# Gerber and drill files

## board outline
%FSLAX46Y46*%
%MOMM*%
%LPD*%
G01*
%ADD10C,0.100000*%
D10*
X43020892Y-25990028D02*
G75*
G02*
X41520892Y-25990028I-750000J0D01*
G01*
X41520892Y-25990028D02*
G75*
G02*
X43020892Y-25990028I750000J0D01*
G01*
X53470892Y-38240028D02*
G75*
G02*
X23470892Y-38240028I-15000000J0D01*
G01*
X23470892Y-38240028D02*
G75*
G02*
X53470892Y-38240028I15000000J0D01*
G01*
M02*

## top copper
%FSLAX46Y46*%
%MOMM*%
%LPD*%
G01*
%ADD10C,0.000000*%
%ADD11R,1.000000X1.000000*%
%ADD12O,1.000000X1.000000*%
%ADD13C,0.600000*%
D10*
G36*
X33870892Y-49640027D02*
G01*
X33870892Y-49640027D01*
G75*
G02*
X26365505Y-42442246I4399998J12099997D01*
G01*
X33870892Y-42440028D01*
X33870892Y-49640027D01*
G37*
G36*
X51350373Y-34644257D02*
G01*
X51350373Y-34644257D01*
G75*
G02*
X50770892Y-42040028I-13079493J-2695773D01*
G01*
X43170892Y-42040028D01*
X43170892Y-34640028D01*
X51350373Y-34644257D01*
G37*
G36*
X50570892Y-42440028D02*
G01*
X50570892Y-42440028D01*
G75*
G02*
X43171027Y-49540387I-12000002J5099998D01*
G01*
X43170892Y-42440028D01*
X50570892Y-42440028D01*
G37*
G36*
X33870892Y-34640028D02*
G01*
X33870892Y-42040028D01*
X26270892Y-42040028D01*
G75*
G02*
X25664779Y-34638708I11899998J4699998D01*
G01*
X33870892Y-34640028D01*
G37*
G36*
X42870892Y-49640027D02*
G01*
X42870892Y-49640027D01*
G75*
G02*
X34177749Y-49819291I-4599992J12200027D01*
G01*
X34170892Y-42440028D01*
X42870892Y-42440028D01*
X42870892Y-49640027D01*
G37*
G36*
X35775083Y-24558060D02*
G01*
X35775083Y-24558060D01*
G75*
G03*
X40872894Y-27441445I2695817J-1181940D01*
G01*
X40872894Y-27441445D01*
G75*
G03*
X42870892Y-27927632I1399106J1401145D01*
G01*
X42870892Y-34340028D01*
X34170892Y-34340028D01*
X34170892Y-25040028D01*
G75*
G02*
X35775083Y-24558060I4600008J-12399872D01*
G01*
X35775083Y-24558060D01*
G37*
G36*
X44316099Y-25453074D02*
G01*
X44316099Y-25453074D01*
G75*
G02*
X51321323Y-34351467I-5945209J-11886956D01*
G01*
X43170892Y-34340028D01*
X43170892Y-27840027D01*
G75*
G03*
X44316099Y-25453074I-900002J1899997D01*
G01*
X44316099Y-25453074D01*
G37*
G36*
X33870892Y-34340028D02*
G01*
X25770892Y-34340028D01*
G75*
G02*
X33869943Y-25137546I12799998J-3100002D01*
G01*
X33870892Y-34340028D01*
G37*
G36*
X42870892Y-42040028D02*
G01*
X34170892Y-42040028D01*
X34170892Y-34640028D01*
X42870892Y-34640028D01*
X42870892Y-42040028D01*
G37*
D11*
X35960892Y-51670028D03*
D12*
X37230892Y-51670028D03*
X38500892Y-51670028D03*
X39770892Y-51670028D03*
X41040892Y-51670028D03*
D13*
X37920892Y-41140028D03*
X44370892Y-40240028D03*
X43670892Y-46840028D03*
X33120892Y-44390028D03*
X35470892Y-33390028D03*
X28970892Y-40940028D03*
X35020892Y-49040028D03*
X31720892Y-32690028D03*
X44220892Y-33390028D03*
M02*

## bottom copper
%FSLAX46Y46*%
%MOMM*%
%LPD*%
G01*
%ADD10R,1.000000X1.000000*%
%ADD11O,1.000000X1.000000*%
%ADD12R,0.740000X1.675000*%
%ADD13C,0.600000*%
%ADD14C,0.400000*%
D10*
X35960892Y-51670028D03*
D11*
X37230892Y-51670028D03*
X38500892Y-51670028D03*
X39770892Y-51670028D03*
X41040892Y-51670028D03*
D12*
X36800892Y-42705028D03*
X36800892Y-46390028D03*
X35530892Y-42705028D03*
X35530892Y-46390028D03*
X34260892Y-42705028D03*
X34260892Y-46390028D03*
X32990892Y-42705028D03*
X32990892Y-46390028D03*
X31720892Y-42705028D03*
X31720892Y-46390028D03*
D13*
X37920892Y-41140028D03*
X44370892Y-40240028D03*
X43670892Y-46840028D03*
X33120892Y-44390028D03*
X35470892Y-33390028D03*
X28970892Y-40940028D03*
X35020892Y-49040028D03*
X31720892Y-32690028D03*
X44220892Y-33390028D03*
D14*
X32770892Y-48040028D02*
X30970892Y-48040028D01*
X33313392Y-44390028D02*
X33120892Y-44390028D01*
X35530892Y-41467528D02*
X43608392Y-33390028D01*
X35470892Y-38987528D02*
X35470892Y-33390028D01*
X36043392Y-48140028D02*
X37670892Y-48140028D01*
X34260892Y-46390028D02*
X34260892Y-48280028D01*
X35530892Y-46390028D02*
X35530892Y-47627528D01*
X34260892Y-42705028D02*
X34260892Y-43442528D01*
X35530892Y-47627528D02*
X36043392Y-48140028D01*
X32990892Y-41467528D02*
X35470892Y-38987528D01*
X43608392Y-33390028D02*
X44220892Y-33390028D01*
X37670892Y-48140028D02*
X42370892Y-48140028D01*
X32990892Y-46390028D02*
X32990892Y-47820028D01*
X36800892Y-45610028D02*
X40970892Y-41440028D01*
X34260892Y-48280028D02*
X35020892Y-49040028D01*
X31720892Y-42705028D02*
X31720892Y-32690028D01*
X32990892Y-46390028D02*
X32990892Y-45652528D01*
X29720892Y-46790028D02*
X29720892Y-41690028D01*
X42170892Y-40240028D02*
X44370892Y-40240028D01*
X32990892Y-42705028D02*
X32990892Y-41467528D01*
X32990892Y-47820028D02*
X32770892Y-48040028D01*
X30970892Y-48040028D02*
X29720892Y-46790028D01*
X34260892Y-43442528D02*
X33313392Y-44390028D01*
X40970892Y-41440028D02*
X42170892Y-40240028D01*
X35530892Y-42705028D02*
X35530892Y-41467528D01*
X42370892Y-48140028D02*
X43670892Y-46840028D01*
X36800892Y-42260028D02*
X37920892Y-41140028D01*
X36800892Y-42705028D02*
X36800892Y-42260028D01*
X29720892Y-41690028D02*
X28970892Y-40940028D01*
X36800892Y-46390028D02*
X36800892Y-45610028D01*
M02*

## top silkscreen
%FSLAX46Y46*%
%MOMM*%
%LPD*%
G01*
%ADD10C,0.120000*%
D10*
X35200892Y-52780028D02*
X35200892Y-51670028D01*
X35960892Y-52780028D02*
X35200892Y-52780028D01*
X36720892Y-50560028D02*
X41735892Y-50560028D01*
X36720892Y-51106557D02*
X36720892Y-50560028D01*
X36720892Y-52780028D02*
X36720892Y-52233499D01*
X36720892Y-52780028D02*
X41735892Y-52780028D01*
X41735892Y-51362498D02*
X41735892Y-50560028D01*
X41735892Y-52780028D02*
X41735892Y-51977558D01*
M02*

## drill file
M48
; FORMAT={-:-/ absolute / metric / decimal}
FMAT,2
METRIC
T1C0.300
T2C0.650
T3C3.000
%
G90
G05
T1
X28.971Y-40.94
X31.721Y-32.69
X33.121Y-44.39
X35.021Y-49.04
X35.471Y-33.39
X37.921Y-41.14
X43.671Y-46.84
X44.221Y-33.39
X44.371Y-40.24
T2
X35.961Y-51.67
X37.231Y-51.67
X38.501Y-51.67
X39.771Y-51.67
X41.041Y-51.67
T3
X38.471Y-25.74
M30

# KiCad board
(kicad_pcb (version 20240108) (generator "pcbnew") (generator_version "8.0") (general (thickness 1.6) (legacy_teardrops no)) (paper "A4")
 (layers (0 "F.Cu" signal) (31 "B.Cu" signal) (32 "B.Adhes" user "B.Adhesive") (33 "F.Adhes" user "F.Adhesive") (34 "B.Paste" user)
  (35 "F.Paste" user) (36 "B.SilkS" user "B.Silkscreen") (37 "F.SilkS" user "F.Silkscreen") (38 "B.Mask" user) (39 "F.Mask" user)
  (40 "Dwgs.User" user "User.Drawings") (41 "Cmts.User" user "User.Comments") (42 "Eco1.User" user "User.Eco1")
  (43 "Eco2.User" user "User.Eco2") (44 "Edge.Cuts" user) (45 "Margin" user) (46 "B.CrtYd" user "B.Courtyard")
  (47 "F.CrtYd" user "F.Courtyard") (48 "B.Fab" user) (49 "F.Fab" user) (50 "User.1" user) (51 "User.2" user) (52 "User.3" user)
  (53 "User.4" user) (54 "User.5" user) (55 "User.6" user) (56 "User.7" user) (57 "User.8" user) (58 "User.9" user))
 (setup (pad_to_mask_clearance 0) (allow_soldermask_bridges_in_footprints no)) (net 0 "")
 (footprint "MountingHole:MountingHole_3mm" (layer "F.Cu") (at 38.470892 25.740028)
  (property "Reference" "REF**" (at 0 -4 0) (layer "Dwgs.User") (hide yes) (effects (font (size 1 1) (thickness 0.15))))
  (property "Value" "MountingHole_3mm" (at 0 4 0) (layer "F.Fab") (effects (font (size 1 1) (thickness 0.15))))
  (pad "" np_thru_hole circle (at 0 0) (size 3 3) (drill 3) (layers "*.Cu" "*.Mask")))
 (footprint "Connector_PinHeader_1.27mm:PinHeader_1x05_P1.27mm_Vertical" (layer "F.Cu") (at 35.960892 51.670028 90)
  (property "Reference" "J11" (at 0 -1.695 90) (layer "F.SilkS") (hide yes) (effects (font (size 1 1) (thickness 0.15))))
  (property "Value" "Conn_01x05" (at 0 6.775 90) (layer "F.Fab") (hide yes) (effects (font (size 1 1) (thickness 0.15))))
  (fp_line (start -1.11 -0.76) (end 0 -0.76) (stroke (width 0.12) (type solid)) (layer "F.SilkS"))
  (fp_line (start -1.11 0) (end -1.11 -0.76) (stroke (width 0.12) (type solid)) (layer "F.SilkS"))
  (fp_line (start 1.11 0.76) (end 1.11 5.775) (stroke (width 0.12) (type solid)) (layer "F.SilkS"))
  (fp_line (start 0.563471 0.76) (end 1.11 0.76) (stroke (width 0.12) (type solid)) (layer "F.SilkS"))
  (fp_line (start -1.11 0.76) (end -0.563471 0.76) (stroke (width 0.12) (type solid)) (layer "F.SilkS"))
  (fp_line (start -1.11 0.76) (end -1.11 5.775) (stroke (width 0.12) (type solid)) (layer "F.SilkS"))
  (fp_line (start 0.30753 5.775) (end 1.11 5.775) (stroke (width 0.12) (type solid)) (layer "F.SilkS"))
  (fp_line (start -1.11 5.775) (end -0.30753 5.775) (stroke (width 0.12) (type solid)) (layer "F.SilkS"))
  (pad "1" thru_hole rect (at 0 0 90) (size 1 1) (drill 0.65) (layers "*.Cu" "*.Mask") (remove_unused_layers no))
  (pad "2" thru_hole oval (at 0 1.27 90) (size 1 1) (drill 0.65) (layers "*.Cu" "*.Mask") (remove_unused_layers no))
  (pad "3" thru_hole oval (at 0 2.54 90) (size 1 1) (drill 0.65) (layers "*.Cu" "*.Mask") (remove_unused_layers no))
  (pad "4" thru_hole oval (at 0 3.81 90) (size 1 1) (drill 0.65) (layers "*.Cu" "*.Mask") (remove_unused_layers no))
  (pad "5" thru_hole oval (at 0 5.08 90) (size 1 1) (drill 0.65) (layers "*.Cu" "*.Mask") (remove_unused_layers no)))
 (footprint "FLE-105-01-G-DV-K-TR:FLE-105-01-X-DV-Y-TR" (layer "B.Cu") (at 34.260892 44.547528 180)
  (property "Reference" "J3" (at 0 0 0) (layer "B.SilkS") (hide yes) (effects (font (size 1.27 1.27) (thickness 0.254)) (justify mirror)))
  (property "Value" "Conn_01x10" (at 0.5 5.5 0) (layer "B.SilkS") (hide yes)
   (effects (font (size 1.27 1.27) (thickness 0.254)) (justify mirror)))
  (pad "1" smd rect (at -2.54 1.8425 180) (size 0.74 1.675) (layers "B.Cu" "B.Paste" "B.Mask"))
  (pad "2" smd rect (at -2.54 -1.8425 180) (size 0.74 1.675) (layers "B.Cu" "B.Paste" "B.Mask"))
  (pad "3" smd rect (at -1.27 1.8425 180) (size 0.74 1.675) (layers "B.Cu" "B.Paste" "B.Mask"))
  (pad "4" smd rect (at -1.27 -1.8425 180) (size 0.74 1.675) (layers "B.Cu" "B.Paste" "B.Mask"))
  (pad "5" smd rect (at 0 1.8425 180) (size 0.74 1.675) (layers "B.Cu" "B.Paste" "B.Mask"))
  (pad "6" smd rect (at 0 -1.8425 180) (size 0.74 1.675) (layers "B.Cu" "B.Paste" "B.Mask"))
  (pad "7" smd rect (at 1.27 1.8425 180) (size 0.74 1.675) (layers "B.Cu" "B.Paste" "B.Mask"))
  (pad "8" smd rect (at 1.27 -1.8425 180) (size 0.74 1.675) (layers "B.Cu" "B.Paste" "B.Mask"))
  (pad "9" smd rect (at 2.54 1.8425 180) (size 0.74 1.675) (layers "B.Cu" "B.Paste" "B.Mask"))
  (pad "10" smd rect (at 2.54 -1.8425 180) (size 0.74 1.675) (layers "B.Cu" "B.Paste" "B.Mask")))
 (gr_poly
  (pts (arc (start 26.365505 42.442246) (mid 29.359191 46.832582) (end 33.870892 49.640027)) (xy 33.870892 42.440028))
  (stroke (width 0) (type solid)) (fill solid) (layer "F.Cu"))
 (gr_poly
  (pts (xy 43.170892 42.040028) (xy 43.170892 34.640028)
   (arc (start 51.350373 34.644257) (mid 51.584487 38.383188) (end 50.770892 42.040028)))
  (stroke (width 0) (type solid)) (fill solid) (layer "F.Cu"))
 (gr_poly
  (pts (arc (start 50.570892 42.440028) (mid 47.598344 46.748275) (end 43.171027 49.540387)) (xy 43.170892 42.440028))
  (stroke (width 0) (type solid)) (fill solid) (layer "F.Cu"))
 (gr_poly
  (pts
   (arc (start 25.664779 34.638708) (mid 25.41905 38.384309) (end 26.270892 42.040028)) (xy 33.870892 42.040028) (xy 33.870892 34.640028))
  (stroke (width 0) (type solid)) (fill solid) (layer "F.Cu"))
 (gr_poly
  (pts
   (arc (start 34.177749 49.819291) (mid 38.539704 50.475661) (end 42.870892 49.640027)) (xy 42.870892 42.440028) (xy 34.170892 42.440028))
  (stroke (width 0) (type solid)) (fill solid) (layer "F.Cu"))
 (gr_poly
  (pts
   (arc (start 35.775083 24.55806) (mid 34.96535 24.773622) (end 34.170892 25.040028)) (xy 34.170892 34.340028) (xy 42.870892 34.340028)
   (arc (start 42.870892 27.927632) (mid 41.803833 27.964233) (end 40.872894 27.441445))
   (arc (start 40.872894 27.441445) (mid 37.021734 28.302131) (end 35.775083 24.55806)))
  (stroke (width 0) (type solid)) (fill solid) (layer "F.Cu"))
 (gr_poly
  (pts
   (arc (start 51.321323 34.351467) (mid 48.81391 29.118804) (end 44.316099 25.453074))
   (arc (start 44.316099 25.453074) (mid 44.166399 26.84945) (end 43.170892 27.840027)) (xy 43.170892 34.340028))
  (stroke (width 0) (type solid)) (fill solid) (layer "F.Cu"))
 (gr_poly
  (pts (arc (start 33.869943 25.137546) (mid 28.684425 28.739007) (end 25.770892 34.340028)) (xy 33.870892 34.340028))
  (stroke (width 0) (type solid)) (fill solid) (layer "F.Cu"))
 (gr_poly
  (pts (xy 42.870892 42.040028) (xy 42.870892 34.640028) (xy 34.170892 34.640028) (xy 34.170892 42.040028)) (stroke (width 0) (type solid))
  (fill solid) (layer "F.Cu"))
 (gr_circle (center 42.270892 25.990028) (end 43.020892 25.990028) (stroke (width 0.1) (type default)) (fill none) (layer "Edge.Cuts"))
 (gr_circle (center 38.470892 38.240028) (end 53.470892 38.240028) (stroke (width 0.1) (type default)) (fill none) (layer "Edge.Cuts"))
 (via (at 37.920892 41.140028) (size 0.6) (drill 0.3) (layers "F.Cu" "B.Cu") (remove_unused_layers yes) (keep_end_layers yes)
  (zone_layer_connections) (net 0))
 (via (at 44.370892 40.240028) (size 0.6) (drill 0.3) (layers "F.Cu" "B.Cu") (remove_unused_layers yes) (keep_end_layers yes)
  (zone_layer_connections) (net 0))
 (via (at 43.670892 46.840028) (size 0.6) (drill 0.3) (layers "F.Cu" "B.Cu") (remove_unused_layers yes) (keep_end_layers yes)
  (zone_layer_connections) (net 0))
 (via (at 33.120892 44.390028) (size 0.6) (drill 0.3) (layers "F.Cu" "B.Cu") (remove_unused_layers yes) (keep_end_layers yes)
  (zone_layer_connections) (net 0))
 (via (at 35.470892 33.390028) (size 0.6) (drill 0.3) (layers "F.Cu" "B.Cu") (remove_unused_layers yes) (keep_end_layers yes)
  (zone_layer_connections) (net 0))
 (via (at 28.970892 40.940028) (size 0.6) (drill 0.3) (layers "F.Cu" "B.Cu") (remove_unused_layers yes) (keep_end_layers yes)
  (zone_layer_connections) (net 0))
 (via (at 35.020892 49.040028) (size 0.6) (drill 0.3) (layers "F.Cu" "B.Cu") (remove_unused_layers yes) (keep_end_layers yes)
  (zone_layer_connections) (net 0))
 (via (at 31.720892 32.690028) (size 0.6) (drill 0.3) (layers "F.Cu" "B.Cu") (remove_unused_layers yes) (keep_end_layers yes)
  (zone_layer_connections) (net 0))
 (via (at 44.220892 33.390028) (size 0.6) (drill 0.3) (layers "F.Cu" "B.Cu") (remove_unused_layers yes) (keep_end_layers yes)
  (zone_layer_connections) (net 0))
 (segment (start 32.770892 48.040028) (end 30.970892 48.040028) (width 0.4) (layer "B.Cu") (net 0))
 (segment (start 33.313392 44.390028) (end 33.120892 44.390028) (width 0.4) (layer "B.Cu") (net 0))
 (segment (start 35.530892 41.467528) (end 43.608392 33.390028) (width 0.4) (layer "B.Cu") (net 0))
 (segment (start 35.470892 38.987528) (end 35.470892 33.390028) (width 0.4) (layer "B.Cu") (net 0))
 (segment (start 36.043392 48.140028) (end 37.670892 48.140028) (width 0.4) (layer "B.Cu") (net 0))
 (segment (start 34.260892 46.390028) (end 34.260892 48.280028) (width 0.4) (layer "B.Cu") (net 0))
 (segment (start 35.530892 46.390028) (end 35.530892 47.627528) (width 0.4) (layer "B.Cu") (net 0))
 (segment (start 34.260892 42.705028) (end 34.260892 43.442528) (width 0.4) (layer "B.Cu") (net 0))
 (segment (start 35.530892 47.627528) (end 36.043392 48.140028) (width 0.4) (layer "B.Cu") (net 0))
 (segment (start 32.990892 41.467528) (end 35.470892 38.987528) (width 0.4) (layer "B.Cu") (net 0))
 (segment (start 43.608392 33.390028) (end 44.220892 33.390028) (width 0.4) (layer "B.Cu") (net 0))
 (segment (start 37.670892 48.140028) (end 42.370892 48.140028) (width 0.4) (layer "B.Cu") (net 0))
 (segment (start 32.990892 46.390028) (end 32.990892 47.820028) (width 0.4) (layer "B.Cu") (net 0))
 (segment (start 36.800892 45.610028) (end 40.970892 41.440028) (width 0.4) (layer "B.Cu") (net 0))
 (segment (start 34.260892 48.280028) (end 35.020892 49.040028) (width 0.4) (layer "B.Cu") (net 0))
 (segment (start 31.720892 42.705028) (end 31.720892 32.690028) (width 0.4) (layer "B.Cu") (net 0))
 (segment (start 32.990892 46.390028) (end 32.990892 45.652528) (width 0.4) (layer "B.Cu") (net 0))
 (segment (start 29.720892 46.790028) (end 29.720892 41.690028) (width 0.4) (layer "B.Cu") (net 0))
 (segment (start 42.170892 40.240028) (end 44.370892 40.240028) (width 0.4) (layer "B.Cu") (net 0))
 (segment (start 32.990892 42.705028) (end 32.990892 41.467528) (width 0.4) (layer "B.Cu") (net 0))
 (segment (start 32.990892 47.820028) (end 32.770892 48.040028) (width 0.4) (layer "B.Cu") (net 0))
 (segment (start 30.970892 48.040028) (end 29.720892 46.790028) (width 0.4) (layer "B.Cu") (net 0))
 (segment (start 34.260892 43.442528) (end 33.313392 44.390028) (width 0.4) (layer "B.Cu") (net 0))
 (segment (start 40.970892 41.440028) (end 42.170892 40.240028) (width 0.4) (layer "B.Cu") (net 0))
 (segment (start 35.530892 42.705028) (end 35.530892 41.467528) (width 0.4) (layer "B.Cu") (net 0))
 (segment (start 42.370892 48.140028) (end 43.670892 46.840028) (width 0.4) (layer "B.Cu") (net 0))
 (segment (start 36.800892 42.260028) (end 37.920892 41.140028) (width 0.4) (layer "B.Cu") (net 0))
 (segment (start 36.800892 42.705028) (end 36.800892 42.260028) (width 0.4) (layer "B.Cu") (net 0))
 (segment (start 29.720892 41.690028) (end 28.970892 40.940028) (width 0.4) (layer "B.Cu") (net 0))
 (segment (start 36.800892 46.390028) (end 36.800892 45.610028) (width 0.4) (layer "B.Cu") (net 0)))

